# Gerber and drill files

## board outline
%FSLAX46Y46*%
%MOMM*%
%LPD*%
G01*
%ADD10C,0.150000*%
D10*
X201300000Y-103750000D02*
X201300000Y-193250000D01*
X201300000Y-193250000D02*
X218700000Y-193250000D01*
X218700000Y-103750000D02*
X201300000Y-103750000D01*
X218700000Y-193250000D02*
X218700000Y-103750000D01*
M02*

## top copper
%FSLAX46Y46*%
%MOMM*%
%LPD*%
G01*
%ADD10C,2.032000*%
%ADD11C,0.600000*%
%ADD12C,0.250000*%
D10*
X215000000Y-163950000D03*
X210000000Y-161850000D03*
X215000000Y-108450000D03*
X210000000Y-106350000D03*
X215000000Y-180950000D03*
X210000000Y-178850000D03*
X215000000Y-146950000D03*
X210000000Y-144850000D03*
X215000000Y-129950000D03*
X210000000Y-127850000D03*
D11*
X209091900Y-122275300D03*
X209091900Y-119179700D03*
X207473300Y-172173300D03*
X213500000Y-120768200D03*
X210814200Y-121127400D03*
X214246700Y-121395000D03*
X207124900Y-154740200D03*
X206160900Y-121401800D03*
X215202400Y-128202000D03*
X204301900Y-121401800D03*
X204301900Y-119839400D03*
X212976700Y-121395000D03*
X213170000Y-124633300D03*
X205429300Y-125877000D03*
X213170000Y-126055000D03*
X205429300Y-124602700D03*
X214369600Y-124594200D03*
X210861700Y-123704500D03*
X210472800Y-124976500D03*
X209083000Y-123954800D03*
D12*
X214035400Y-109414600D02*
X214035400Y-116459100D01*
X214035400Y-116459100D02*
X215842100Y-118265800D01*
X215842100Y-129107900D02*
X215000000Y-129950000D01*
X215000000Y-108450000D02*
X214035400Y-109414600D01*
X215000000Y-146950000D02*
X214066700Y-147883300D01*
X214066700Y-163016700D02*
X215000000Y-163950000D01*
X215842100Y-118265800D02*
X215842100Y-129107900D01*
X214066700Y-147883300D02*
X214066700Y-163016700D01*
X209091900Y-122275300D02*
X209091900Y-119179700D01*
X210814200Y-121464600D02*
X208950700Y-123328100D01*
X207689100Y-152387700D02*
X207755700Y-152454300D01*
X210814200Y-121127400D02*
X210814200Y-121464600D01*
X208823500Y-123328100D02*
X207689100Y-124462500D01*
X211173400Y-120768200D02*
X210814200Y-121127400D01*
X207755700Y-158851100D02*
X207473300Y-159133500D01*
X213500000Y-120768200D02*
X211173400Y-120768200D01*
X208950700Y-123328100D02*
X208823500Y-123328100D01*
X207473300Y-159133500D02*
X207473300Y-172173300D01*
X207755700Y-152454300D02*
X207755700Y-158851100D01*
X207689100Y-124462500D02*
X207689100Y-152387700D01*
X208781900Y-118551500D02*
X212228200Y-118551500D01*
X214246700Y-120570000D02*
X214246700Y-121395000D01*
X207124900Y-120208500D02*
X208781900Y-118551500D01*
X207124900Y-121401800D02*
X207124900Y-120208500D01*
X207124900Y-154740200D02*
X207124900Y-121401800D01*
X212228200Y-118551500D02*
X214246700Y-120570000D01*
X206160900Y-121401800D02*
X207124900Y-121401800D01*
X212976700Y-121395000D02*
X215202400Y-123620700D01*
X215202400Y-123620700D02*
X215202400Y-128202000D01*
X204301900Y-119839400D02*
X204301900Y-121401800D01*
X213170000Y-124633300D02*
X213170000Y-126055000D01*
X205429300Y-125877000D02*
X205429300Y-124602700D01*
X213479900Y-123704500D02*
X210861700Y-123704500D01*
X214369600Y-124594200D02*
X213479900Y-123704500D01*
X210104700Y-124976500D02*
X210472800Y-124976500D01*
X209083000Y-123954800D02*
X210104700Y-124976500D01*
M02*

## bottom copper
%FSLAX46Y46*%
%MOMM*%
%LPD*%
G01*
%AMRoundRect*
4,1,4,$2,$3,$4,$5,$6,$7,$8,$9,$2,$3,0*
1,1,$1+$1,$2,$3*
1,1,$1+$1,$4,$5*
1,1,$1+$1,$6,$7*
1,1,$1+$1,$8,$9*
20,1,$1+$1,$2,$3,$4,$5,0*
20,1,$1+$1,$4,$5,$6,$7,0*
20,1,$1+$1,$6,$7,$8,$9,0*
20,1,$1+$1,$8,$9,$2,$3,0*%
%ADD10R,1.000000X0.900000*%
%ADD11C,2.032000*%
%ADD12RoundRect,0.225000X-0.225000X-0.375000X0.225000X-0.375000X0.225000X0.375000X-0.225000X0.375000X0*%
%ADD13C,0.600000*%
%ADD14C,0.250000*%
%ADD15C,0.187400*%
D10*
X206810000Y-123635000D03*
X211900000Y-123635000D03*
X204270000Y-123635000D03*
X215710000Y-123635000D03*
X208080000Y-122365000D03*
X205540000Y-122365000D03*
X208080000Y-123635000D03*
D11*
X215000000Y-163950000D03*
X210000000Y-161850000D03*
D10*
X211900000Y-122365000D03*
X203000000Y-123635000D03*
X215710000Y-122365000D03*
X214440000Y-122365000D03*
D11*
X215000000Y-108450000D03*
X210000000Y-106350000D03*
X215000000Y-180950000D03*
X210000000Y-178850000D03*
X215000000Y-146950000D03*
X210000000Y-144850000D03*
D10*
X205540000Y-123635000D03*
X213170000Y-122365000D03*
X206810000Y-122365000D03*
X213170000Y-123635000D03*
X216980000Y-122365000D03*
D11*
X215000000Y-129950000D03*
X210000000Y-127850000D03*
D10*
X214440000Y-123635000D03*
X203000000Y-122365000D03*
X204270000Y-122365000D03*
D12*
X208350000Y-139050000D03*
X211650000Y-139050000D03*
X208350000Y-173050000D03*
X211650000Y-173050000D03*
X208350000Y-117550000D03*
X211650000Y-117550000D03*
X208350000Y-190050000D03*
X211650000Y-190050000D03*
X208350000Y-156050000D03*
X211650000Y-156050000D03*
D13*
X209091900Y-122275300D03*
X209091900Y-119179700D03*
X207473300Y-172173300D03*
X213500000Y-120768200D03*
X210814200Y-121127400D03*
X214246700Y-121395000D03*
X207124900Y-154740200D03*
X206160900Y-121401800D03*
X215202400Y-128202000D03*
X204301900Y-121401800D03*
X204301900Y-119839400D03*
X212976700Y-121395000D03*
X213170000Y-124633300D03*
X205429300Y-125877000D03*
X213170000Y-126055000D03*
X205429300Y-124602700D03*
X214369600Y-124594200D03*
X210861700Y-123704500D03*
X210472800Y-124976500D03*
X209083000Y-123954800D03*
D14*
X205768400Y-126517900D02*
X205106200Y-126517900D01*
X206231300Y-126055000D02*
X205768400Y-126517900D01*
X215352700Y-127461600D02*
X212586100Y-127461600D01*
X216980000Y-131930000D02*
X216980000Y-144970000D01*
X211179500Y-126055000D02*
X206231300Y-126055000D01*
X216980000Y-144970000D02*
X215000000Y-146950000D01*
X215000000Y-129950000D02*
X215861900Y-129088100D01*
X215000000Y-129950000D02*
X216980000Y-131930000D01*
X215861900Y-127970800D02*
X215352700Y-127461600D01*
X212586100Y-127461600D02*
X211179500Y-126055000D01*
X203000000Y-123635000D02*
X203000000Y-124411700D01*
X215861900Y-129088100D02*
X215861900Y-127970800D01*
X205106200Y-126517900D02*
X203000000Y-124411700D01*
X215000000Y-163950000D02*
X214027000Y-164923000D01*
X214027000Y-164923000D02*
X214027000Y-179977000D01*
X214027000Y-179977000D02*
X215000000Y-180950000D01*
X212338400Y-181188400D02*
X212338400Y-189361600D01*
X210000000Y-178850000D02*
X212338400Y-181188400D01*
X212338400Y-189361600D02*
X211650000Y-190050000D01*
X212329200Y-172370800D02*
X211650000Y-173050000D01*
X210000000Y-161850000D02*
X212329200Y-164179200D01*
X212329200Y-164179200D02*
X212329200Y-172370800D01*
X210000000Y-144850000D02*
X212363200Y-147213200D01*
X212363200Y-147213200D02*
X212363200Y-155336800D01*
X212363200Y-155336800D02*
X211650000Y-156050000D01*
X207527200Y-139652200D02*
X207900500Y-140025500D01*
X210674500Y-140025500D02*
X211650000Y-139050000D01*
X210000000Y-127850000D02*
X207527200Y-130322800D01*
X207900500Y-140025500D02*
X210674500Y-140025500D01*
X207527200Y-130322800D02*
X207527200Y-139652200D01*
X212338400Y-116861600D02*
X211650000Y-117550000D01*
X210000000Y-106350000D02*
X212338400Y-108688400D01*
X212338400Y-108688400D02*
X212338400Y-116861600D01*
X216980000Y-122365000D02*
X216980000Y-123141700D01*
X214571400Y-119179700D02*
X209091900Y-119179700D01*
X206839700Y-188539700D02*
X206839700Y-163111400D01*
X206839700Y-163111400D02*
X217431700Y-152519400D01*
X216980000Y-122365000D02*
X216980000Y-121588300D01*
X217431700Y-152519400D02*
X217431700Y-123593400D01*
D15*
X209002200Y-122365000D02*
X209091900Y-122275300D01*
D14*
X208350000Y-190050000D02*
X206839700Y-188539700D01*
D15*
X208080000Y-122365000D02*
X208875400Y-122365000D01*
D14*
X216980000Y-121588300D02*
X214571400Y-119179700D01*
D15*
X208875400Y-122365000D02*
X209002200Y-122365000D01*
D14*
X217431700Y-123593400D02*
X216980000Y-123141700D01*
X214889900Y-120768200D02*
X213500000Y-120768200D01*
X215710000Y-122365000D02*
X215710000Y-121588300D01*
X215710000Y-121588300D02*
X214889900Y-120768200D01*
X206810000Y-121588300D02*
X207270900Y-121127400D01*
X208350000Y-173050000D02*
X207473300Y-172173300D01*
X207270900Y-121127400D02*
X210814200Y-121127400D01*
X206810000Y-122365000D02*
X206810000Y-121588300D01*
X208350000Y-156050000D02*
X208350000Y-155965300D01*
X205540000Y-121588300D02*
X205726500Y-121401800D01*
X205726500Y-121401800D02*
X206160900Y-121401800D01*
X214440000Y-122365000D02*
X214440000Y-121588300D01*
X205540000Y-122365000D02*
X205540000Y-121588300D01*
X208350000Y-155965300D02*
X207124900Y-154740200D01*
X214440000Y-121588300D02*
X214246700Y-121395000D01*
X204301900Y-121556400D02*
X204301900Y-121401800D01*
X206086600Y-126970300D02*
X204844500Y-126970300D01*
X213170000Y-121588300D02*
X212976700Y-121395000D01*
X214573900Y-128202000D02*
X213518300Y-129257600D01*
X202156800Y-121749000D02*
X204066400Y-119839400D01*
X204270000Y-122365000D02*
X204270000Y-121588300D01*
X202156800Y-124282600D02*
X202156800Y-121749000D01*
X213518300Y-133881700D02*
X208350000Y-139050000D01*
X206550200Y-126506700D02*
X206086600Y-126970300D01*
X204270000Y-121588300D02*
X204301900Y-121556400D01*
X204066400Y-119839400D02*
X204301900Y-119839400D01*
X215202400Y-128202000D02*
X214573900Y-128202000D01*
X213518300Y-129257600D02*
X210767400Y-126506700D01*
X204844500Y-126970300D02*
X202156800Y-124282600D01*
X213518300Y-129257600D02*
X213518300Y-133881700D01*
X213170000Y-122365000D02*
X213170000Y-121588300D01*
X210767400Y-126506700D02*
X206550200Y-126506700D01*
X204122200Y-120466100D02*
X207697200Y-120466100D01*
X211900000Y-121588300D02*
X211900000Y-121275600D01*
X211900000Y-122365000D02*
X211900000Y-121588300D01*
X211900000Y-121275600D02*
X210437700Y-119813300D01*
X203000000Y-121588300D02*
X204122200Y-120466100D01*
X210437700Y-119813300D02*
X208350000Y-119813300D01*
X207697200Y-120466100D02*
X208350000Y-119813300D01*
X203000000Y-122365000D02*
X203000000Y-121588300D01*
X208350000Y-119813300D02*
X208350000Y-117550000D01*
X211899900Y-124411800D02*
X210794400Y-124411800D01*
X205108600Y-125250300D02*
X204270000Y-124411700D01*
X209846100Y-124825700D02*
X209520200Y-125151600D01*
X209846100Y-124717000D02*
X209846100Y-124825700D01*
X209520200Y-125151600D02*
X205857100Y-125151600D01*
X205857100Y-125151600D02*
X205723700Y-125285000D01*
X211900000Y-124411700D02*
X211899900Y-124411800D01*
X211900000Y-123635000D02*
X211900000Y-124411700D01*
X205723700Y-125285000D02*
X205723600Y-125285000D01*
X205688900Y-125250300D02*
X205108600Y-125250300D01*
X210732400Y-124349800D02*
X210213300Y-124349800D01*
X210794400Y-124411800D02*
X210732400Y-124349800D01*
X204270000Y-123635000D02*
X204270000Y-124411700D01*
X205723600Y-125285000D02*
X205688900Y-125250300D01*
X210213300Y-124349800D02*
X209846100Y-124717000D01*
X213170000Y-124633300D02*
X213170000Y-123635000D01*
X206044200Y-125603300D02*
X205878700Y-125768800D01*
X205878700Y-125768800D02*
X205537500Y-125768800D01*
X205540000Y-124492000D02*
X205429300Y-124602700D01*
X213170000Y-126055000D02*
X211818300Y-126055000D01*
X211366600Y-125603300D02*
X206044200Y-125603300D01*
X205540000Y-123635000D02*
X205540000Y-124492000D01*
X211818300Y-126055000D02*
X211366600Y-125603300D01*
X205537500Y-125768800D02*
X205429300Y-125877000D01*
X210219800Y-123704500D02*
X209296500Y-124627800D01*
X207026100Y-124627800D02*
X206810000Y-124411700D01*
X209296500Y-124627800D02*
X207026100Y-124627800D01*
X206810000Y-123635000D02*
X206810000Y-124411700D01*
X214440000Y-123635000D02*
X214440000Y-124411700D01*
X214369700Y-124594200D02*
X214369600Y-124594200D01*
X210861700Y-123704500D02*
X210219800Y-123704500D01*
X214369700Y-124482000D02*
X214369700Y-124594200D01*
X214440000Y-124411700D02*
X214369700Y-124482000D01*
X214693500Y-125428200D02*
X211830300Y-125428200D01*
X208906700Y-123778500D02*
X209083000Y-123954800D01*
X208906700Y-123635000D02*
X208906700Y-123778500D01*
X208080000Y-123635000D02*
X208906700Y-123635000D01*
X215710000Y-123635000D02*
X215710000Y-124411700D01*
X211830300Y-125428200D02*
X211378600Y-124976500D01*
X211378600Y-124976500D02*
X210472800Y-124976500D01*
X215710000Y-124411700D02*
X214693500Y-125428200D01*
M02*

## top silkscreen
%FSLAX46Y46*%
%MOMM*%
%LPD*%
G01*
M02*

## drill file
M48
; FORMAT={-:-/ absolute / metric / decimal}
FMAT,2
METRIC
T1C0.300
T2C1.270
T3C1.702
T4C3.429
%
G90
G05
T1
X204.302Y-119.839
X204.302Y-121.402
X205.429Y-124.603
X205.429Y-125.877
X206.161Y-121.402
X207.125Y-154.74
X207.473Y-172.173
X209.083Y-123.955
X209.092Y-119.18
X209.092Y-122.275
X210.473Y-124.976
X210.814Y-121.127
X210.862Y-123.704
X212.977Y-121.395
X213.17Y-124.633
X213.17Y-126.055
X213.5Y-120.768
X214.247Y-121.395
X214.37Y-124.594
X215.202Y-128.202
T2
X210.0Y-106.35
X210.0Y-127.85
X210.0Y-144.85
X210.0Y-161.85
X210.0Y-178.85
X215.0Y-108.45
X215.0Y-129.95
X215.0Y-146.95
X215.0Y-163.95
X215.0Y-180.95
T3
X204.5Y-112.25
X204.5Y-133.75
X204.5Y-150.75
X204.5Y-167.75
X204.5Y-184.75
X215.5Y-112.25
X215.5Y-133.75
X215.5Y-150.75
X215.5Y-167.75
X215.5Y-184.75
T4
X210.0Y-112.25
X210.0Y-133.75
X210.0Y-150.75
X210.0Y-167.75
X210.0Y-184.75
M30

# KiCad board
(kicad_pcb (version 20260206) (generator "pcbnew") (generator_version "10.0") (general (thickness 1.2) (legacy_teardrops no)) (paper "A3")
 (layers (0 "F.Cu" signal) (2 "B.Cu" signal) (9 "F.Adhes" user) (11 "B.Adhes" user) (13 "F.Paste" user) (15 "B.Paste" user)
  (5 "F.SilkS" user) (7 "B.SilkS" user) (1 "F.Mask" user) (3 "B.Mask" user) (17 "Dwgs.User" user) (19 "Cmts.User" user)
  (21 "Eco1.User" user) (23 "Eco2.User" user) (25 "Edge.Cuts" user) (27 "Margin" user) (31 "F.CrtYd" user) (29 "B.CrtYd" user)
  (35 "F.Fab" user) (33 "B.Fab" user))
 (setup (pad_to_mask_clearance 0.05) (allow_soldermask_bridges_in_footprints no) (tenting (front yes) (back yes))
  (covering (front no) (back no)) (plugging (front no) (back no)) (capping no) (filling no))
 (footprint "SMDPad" (layer "F.Cu") (at 206.81 123.635)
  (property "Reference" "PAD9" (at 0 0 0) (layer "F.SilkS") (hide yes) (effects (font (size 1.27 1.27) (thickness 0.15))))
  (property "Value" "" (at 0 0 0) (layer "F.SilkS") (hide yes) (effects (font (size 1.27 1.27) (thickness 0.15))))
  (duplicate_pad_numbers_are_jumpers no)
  (pad "1" smd rect (at 0 0) (size 1 0.9) (layers "B.Cu" "B.Mask" "B.Paste") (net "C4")))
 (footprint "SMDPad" (layer "F.Cu") (at 211.9 123.635)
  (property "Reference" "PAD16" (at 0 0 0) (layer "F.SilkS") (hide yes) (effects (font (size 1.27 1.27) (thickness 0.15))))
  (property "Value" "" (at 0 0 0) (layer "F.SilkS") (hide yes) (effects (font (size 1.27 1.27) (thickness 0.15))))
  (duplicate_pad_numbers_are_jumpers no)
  (pad "1" smd rect (at 0 0) (size 1 0.9) (layers "B.Cu" "B.Mask" "B.Paste") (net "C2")))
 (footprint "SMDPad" (layer "F.Cu") (at 204.27 123.635)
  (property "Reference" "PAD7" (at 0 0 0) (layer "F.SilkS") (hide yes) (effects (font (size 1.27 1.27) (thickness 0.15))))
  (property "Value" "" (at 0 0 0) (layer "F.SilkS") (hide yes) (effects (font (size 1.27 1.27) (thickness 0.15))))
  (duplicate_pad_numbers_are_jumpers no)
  (pad "1" smd rect (at 0 0) (size 1 0.9) (layers "B.Cu" "B.Mask" "B.Paste") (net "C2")))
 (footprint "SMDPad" (layer "F.Cu") (at 215.71 123.635)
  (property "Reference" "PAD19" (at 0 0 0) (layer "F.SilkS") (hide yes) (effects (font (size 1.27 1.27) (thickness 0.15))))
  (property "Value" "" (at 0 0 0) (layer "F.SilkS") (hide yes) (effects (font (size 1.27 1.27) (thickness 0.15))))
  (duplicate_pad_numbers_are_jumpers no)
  (pad "1" smd rect (at 0 0) (size 1 0.9) (layers "B.Cu" "B.Mask" "B.Paste") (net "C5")))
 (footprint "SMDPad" (layer "F.Cu") (at 208.08 122.365)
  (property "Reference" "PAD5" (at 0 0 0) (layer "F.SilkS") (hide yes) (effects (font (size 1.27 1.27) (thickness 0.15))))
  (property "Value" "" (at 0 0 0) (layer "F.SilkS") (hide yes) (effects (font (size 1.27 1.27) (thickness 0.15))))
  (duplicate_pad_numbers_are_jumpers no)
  (pad "1" smd rect (at 0 0) (size 1 0.9) (layers "B.Cu" "B.Mask" "B.Paste") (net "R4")))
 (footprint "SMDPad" (layer "F.Cu") (at 205.54 122.365)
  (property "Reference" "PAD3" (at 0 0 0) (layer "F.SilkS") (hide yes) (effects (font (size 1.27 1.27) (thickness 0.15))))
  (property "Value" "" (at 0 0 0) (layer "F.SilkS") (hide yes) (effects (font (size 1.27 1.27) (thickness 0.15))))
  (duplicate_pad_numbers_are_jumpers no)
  (pad "1" smd rect (at 0 0) (size 1 0.9) (layers "B.Cu" "B.Mask" "B.Paste") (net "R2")))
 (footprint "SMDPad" (layer "F.Cu") (at 208.08 123.635)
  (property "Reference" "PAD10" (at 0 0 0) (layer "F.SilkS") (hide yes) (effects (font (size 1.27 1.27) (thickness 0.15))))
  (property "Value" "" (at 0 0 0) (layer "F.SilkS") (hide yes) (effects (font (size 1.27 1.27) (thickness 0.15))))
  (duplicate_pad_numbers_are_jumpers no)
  (pad "1" smd rect (at 0 0) (size 1 0.9) (layers "B.Cu" "B.Mask" "B.Paste") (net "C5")))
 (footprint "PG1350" (layer "F.Cu") (at 210 167.75)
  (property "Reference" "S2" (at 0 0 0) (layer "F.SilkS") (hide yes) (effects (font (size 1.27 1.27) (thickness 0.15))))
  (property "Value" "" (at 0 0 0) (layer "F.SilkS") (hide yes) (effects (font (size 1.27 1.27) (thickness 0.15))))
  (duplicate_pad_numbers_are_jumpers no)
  (pad "" np_thru_hole circle (at -5.5 0) (size 1.7018 1.7018) (drill 1.7018) (layers "*.Cu" "*.Mask"))
  (pad "" np_thru_hole circle (at 0 0) (size 3.429 3.429) (drill 3.429) (layers "*.Cu" "*.Mask"))
  (pad "" np_thru_hole circle (at 5.5 0) (size 1.7018 1.7018) (drill 1.7018) (layers "*.Cu" "*.Mask"))
  (pad "1" thru_hole circle (at 5 -3.8) (size 2.032 2.032) (drill 1.27) (layers "*.Cu" "*.Mask") (remove_unused_layers no) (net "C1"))
  (pad "2" thru_hole circle (at 0 -5.9) (size 2.032 2.032) (drill 1.27) (layers "*.Cu" "*.Mask") (remove_unused_layers no) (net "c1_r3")))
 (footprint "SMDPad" (layer "F.Cu") (at 211.9 122.365)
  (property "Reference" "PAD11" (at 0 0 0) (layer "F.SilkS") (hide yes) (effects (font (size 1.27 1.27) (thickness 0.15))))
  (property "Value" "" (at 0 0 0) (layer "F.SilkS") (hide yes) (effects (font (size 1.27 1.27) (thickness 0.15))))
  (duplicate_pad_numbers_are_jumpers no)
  (pad "1" smd rect (at 0 0) (size 1 0.9) (layers "B.Cu" "B.Mask" "B.Paste") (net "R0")))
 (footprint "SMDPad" (layer "F.Cu") (at 203 123.635)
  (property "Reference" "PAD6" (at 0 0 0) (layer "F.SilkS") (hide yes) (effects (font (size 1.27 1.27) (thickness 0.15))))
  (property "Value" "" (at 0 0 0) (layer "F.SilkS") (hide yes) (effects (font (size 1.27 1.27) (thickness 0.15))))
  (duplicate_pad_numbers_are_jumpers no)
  (pad "1" smd rect (at 0 0) (size 1 0.9) (layers "B.Cu" "B.Mask" "B.Paste") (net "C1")))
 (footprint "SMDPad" (layer "F.Cu") (at 215.71 122.365)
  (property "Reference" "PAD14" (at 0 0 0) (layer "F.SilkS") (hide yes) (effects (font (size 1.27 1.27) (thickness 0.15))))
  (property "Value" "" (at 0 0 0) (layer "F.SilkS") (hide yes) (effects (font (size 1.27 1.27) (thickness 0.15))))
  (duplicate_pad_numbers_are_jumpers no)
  (pad "1" smd rect (at 0 0) (size 1 0.9) (layers "B.Cu" "B.Mask" "B.Paste") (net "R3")))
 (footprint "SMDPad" (layer "F.Cu") (at 214.44 122.365)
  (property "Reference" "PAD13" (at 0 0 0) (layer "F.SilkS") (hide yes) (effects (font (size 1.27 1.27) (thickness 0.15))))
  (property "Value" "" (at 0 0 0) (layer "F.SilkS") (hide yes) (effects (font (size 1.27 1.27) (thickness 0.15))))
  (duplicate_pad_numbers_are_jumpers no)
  (pad "1" smd rect (at 0 0) (size 1 0.9) (layers "B.Cu" "B.Mask" "B.Paste") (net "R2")))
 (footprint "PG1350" (layer "F.Cu") (at 210 112.25)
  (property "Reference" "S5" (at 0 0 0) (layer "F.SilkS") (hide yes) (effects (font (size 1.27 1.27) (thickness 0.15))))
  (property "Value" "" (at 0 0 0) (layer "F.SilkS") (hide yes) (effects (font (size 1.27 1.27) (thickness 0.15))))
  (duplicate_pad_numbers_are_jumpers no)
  (pad "" np_thru_hole circle (at -5.5 0) (size 1.7018 1.7018) (drill 1.7018) (layers "*.Cu" "*.Mask"))
  (pad "" np_thru_hole circle (at 0 0) (size 3.429 3.429) (drill 3.429) (layers "*.Cu" "*.Mask"))
  (pad "" np_thru_hole circle (at 5.5 0) (size 1.7018 1.7018) (drill 1.7018) (layers "*.Cu" "*.Mask"))
  (pad "1" thru_hole circle (at 5 -3.8) (size 2.032 2.032) (drill 1.27) (layers "*.Cu" "*.Mask") (remove_unused_layers no) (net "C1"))
  (pad "2" thru_hole circle (at 0 -5.9) (size 2.032 2.032) (drill 1.27) (layers "*.Cu" "*.Mask") (remove_unused_layers no) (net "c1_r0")))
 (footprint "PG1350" (layer "F.Cu") (at 210 184.75)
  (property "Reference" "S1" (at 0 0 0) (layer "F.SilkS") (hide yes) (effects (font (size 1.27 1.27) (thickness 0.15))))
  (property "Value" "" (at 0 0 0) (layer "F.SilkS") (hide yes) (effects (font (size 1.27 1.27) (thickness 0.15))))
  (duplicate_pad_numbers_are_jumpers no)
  (pad "" np_thru_hole circle (at -5.5 0) (size 1.7018 1.7018) (drill 1.7018) (layers "*.Cu" "*.Mask"))
  (pad "" np_thru_hole circle (at 0 0) (size 3.429 3.429) (drill 3.429) (layers "*.Cu" "*.Mask"))
  (pad "" np_thru_hole circle (at 5.5 0) (size 1.7018 1.7018) (drill 1.7018) (layers "*.Cu" "*.Mask"))
  (pad "1" thru_hole circle (at 5 -3.8) (size 2.032 2.032) (drill 1.27) (layers "*.Cu" "*.Mask") (remove_unused_layers no) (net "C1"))
  (pad "2" thru_hole circle (at 0 -5.9) (size 2.032 2.032) (drill 1.27) (layers "*.Cu" "*.Mask") (remove_unused_layers no) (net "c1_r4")))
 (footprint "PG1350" (layer "F.Cu") (at 210 150.75)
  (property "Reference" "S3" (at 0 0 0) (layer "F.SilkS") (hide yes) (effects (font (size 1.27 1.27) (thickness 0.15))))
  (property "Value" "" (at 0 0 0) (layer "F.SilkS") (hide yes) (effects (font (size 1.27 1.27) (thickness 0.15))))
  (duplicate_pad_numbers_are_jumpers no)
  (pad "" np_thru_hole circle (at -5.5 0) (size 1.7018 1.7018) (drill 1.7018) (layers "*.Cu" "*.Mask"))
  (pad "" np_thru_hole circle (at 0 0) (size 3.429 3.429) (drill 3.429) (layers "*.Cu" "*.Mask"))
  (pad "" np_thru_hole circle (at 5.5 0) (size 1.7018 1.7018) (drill 1.7018) (layers "*.Cu" "*.Mask"))
  (pad "1" thru_hole circle (at 5 -3.8) (size 2.032 2.032) (drill 1.27) (layers "*.Cu" "*.Mask") (remove_unused_layers no) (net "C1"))
  (pad "2" thru_hole circle (at 0 -5.9) (size 2.032 2.032) (drill 1.27) (layers "*.Cu" "*.Mask") (remove_unused_layers no) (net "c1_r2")))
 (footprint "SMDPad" (layer "F.Cu") (at 205.54 123.635)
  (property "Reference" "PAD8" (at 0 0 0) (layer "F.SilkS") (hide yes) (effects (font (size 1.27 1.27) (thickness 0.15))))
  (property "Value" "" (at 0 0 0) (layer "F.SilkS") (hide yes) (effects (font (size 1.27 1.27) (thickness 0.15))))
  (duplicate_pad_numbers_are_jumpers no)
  (pad "1" smd rect (at 0 0) (size 1 0.9) (layers "B.Cu" "B.Mask" "B.Paste") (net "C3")))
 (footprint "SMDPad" (layer "F.Cu") (at 213.17 122.365)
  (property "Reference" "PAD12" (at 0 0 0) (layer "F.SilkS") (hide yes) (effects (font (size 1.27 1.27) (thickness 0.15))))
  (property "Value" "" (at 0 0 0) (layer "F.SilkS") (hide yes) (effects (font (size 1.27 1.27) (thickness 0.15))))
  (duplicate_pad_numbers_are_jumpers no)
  (pad "1" smd rect (at 0 0) (size 1 0.9) (layers "B.Cu" "B.Mask" "B.Paste") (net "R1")))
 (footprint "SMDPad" (layer "F.Cu") (at 206.81 122.365)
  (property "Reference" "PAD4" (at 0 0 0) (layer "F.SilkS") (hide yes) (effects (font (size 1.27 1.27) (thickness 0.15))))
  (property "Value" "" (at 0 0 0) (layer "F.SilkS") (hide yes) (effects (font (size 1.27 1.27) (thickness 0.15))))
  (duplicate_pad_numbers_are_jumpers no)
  (pad "1" smd rect (at 0 0) (size 1 0.9) (layers "B.Cu" "B.Mask" "B.Paste") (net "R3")))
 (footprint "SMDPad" (layer "F.Cu") (at 213.17 123.635)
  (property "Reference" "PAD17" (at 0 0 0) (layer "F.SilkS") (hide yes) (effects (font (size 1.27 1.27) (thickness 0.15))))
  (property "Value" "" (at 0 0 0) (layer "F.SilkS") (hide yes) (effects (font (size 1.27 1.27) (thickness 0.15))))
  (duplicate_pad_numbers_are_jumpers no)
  (pad "1" smd rect (at 0 0) (size 1 0.9) (layers "B.Cu" "B.Mask" "B.Paste") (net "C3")))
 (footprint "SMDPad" (layer "F.Cu") (at 216.98 122.365)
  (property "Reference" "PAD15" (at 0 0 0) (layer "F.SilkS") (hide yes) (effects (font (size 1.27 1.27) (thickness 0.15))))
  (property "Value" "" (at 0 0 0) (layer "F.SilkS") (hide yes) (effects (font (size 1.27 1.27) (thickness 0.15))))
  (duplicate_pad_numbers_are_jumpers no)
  (pad "1" smd rect (at 0 0) (size 1 0.9) (layers "B.Cu" "B.Mask" "B.Paste") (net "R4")))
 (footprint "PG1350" (layer "F.Cu") (at 210 133.75)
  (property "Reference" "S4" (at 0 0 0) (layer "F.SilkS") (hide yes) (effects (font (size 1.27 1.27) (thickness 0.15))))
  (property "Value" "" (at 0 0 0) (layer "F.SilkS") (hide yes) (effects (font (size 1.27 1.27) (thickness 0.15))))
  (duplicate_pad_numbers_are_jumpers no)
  (pad "" np_thru_hole circle (at -5.5 0) (size 1.7018 1.7018) (drill 1.7018) (layers "*.Cu" "*.Mask"))
  (pad "" np_thru_hole circle (at 0 0) (size 3.429 3.429) (drill 3.429) (layers "*.Cu" "*.Mask"))
  (pad "" np_thru_hole circle (at 5.5 0) (size 1.7018 1.7018) (drill 1.7018) (layers "*.Cu" "*.Mask"))
  (pad "1" thru_hole circle (at 5 -3.8) (size 2.032 2.032) (drill 1.27) (layers "*.Cu" "*.Mask") (remove_unused_layers no) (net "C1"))
  (pad "2" thru_hole circle (at 0 -5.9) (size 2.032 2.032) (drill 1.27) (layers "*.Cu" "*.Mask") (remove_unused_layers no) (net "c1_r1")))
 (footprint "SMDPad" (layer "F.Cu") (at 214.44 123.635)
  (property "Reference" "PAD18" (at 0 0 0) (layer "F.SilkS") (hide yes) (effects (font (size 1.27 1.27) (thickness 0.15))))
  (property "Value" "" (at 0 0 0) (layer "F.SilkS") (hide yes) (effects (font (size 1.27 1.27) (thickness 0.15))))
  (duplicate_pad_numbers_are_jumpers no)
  (pad "1" smd rect (at 0 0) (size 1 0.9) (layers "B.Cu" "B.Mask" "B.Paste") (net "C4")))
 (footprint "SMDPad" (layer "F.Cu") (at 203 122.365)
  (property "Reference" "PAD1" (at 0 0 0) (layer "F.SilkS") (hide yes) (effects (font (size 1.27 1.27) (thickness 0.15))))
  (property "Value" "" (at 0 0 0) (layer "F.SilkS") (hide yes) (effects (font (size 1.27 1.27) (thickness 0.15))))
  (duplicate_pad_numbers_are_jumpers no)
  (pad "1" smd rect (at 0 0) (size 1 0.9) (layers "B.Cu" "B.Mask" "B.Paste") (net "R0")))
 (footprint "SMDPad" (layer "F.Cu") (at 204.27 122.365)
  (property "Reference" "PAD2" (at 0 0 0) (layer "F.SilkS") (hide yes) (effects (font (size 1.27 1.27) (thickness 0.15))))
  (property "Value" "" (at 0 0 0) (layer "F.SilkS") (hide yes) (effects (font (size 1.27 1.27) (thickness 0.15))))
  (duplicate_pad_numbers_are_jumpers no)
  (pad "1" smd rect (at 0 0) (size 1 0.9) (layers "B.Cu" "B.Mask" "B.Paste") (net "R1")))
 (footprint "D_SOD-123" (layer "B.Cu") (at 210 139.05)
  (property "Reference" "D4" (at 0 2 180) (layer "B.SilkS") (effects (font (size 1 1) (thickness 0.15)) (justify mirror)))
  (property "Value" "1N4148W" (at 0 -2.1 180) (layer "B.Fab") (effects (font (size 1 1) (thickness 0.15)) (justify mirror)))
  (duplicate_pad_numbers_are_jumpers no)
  (pad "1" smd roundrect (at -1.65 0) (size 0.9 1.2) (layers "B.Cu" "B.Mask" "B.Paste") (roundrect_rratio 0.25) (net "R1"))
  (pad "2" smd roundrect (at 1.65 0) (size 0.9 1.2) (layers "B.Cu" "B.Mask" "B.Paste") (roundrect_rratio 0.25) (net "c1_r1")))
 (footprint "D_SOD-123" (layer "B.Cu") (at 210 173.05)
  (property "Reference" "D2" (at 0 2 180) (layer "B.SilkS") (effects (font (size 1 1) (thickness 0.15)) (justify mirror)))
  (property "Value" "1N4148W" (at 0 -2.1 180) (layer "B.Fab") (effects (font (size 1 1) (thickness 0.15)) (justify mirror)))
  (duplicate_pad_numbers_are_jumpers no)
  (pad "1" smd roundrect (at -1.65 0) (size 0.9 1.2) (layers "B.Cu" "B.Mask" "B.Paste") (roundrect_rratio 0.25) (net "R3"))
  (pad "2" smd roundrect (at 1.65 0) (size 0.9 1.2) (layers "B.Cu" "B.Mask" "B.Paste") (roundrect_rratio 0.25) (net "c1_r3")))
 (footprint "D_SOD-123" (layer "B.Cu") (at 210 117.55)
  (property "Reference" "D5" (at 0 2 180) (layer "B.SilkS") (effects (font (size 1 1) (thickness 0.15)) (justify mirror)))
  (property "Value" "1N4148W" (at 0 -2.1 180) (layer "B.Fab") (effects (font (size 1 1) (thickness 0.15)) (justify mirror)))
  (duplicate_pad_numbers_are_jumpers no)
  (pad "1" smd roundrect (at -1.65 0) (size 0.9 1.2) (layers "B.Cu" "B.Mask" "B.Paste") (roundrect_rratio 0.25) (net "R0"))
  (pad "2" smd roundrect (at 1.65 0) (size 0.9 1.2) (layers "B.Cu" "B.Mask" "B.Paste") (roundrect_rratio 0.25) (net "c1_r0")))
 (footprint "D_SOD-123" (layer "B.Cu") (at 210 190.05)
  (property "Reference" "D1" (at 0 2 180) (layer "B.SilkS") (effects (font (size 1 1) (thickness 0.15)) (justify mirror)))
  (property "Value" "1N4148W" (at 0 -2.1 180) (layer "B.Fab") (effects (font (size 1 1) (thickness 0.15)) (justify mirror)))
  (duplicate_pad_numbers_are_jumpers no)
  (pad "1" smd roundrect (at -1.65 0) (size 0.9 1.2) (layers "B.Cu" "B.Mask" "B.Paste") (roundrect_rratio 0.25) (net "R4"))
  (pad "2" smd roundrect (at 1.65 0) (size 0.9 1.2) (layers "B.Cu" "B.Mask" "B.Paste") (roundrect_rratio 0.25) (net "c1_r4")))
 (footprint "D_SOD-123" (layer "B.Cu") (at 210 156.05)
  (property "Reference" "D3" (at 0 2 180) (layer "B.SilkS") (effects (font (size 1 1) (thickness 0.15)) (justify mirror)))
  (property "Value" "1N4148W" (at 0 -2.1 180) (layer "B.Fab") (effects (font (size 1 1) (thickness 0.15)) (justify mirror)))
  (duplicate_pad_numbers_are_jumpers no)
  (pad "1" smd roundrect (at -1.65 0) (size 0.9 1.2) (layers "B.Cu" "B.Mask" "B.Paste") (roundrect_rratio 0.25) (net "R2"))
  (pad "2" smd roundrect (at 1.65 0) (size 0.9 1.2) (layers "B.Cu" "B.Mask" "B.Paste") (roundrect_rratio 0.25) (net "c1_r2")))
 (gr_line (start 201.3 103.75) (end 201.3 193.25) (stroke (width 0.15) (type solid)) (layer "Edge.Cuts"))
 (gr_line (start 201.3 193.25) (end 218.7 193.25) (stroke (width 0.15) (type solid)) (layer "Edge.Cuts"))
 (gr_line (start 218.7 103.75) (end 201.3 103.75) (stroke (width 0.15) (type solid)) (layer "Edge.Cuts"))
 (gr_line (start 218.7 193.25) (end 218.7 103.75) (stroke (width 0.15) (type solid)) (layer "Edge.Cuts"))
 (segment (start 214.0354 109.4146) (end 214.0354 116.4591) (width 0.25) (layer "F.Cu") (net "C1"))
 (segment (start 214.0354 116.4591) (end 215.8421 118.2658) (width 0.25) (layer "F.Cu") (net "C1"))
 (segment (start 215.8421 129.1079) (end 215 129.95) (width 0.25) (layer "F.Cu") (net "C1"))
 (segment (start 215 108.45) (end 214.0354 109.4146) (width 0.25) (layer "F.Cu") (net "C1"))
 (segment (start 215 146.95) (end 214.0667 147.8833) (width 0.25) (layer "F.Cu") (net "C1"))
 (segment (start 214.0667 163.0167) (end 215 163.95) (width 0.25) (layer "F.Cu") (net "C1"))
 (segment (start 215.8421 118.2658) (end 215.8421 129.1079) (width 0.25) (layer "F.Cu") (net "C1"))
 (segment (start 214.0667 147.8833) (end 214.0667 163.0167) (width 0.25) (layer "F.Cu") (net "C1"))
 (segment (start 205.7684 126.5179) (end 205.1062 126.5179) (width 0.25) (layer "B.Cu") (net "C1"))
 (segment (start 206.2313 126.055) (end 205.7684 126.5179) (width 0.25) (layer "B.Cu") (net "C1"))
 (segment (start 215.3527 127.4616) (end 212.5861 127.4616) (width 0.25) (layer "B.Cu") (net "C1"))
 (segment (start 216.98 131.93) (end 216.98 144.97) (width 0.25) (layer "B.Cu") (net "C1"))
 (segment (start 211.1795 126.055) (end 206.2313 126.055) (width 0.25) (layer "B.Cu") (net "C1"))
 (segment (start 216.98 144.97) (end 215 146.95) (width 0.25) (layer "B.Cu") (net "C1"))
 (segment (start 215 129.95) (end 215.8619 129.0881) (width 0.25) (layer "B.Cu") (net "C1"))
 (segment (start 215 129.95) (end 216.98 131.93) (width 0.25) (layer "B.Cu") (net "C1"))
 (segment (start 215.8619 127.9708) (end 215.3527 127.4616) (width 0.25) (layer "B.Cu") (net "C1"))
 (segment (start 212.5861 127.4616) (end 211.1795 126.055) (width 0.25) (layer "B.Cu") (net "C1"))
 (segment (start 203 123.635) (end 203 124.4117) (width 0.25) (layer "B.Cu") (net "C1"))
 (segment (start 215.8619 129.0881) (end 215.8619 127.9708) (width 0.25) (layer "B.Cu") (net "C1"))
 (segment (start 205.1062 126.5179) (end 203 124.4117) (width 0.25) (layer "B.Cu") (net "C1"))
 (segment (start 215 163.95) (end 214.027 164.923) (width 0.25) (layer "B.Cu") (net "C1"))
 (segment (start 214.027 164.923) (end 214.027 179.977) (width 0.25) (layer "B.Cu") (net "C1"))
 (segment (start 214.027 179.977) (end 215 180.95) (width 0.25) (layer "B.Cu") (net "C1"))
 (segment (start 212.3384 181.1884) (end 212.3384 189.3616) (width 0.25) (layer "B.Cu") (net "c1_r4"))
 (segment (start 210 178.85) (end 212.3384 181.1884) (width 0.25) (layer "B.Cu") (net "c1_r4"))
 (segment (start 212.3384 189.3616) (end 211.65 190.05) (width 0.25) (layer "B.Cu") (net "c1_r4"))
 (segment (start 212.3292 172.3708) (end 211.65 173.05) (width 0.25) (layer "B.Cu") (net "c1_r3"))
 (segment (start 210 161.85) (end 212.3292 164.1792) (width 0.25) (layer "B.Cu") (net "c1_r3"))
 (segment (start 212.3292 164.1792) (end 212.3292 172.3708) (width 0.25) (layer "B.Cu") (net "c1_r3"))
 (segment (start 210 144.85) (end 212.3632 147.2132) (width 0.25) (layer "B.Cu") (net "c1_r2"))
 (segment (start 212.3632 147.2132) (end 212.3632 155.3368) (width 0.25) (layer "B.Cu") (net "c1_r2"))
 (segment (start 212.3632 155.3368) (end 211.65 156.05) (width 0.25) (layer "B.Cu") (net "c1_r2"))
 (segment (start 207.5272 139.6522) (end 207.9005 140.0255) (width 0.25) (layer "B.Cu") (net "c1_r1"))
 (segment (start 210.6745 140.0255) (end 211.65 139.05) (width 0.25) (layer "B.Cu") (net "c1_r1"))
 (segment (start 210 127.85) (end 207.5272 130.3228) (width 0.25) (layer "B.Cu") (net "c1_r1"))
 (segment (start 207.9005 140.0255) (end 210.6745 140.0255) (width 0.25) (layer "B.Cu") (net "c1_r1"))
 (segment (start 207.5272 130.3228) (end 207.5272 139.6522) (width 0.25) (layer "B.Cu") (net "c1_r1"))
 (segment (start 212.3384 116.8616) (end 211.65 117.55) (width 0.25) (layer "B.Cu") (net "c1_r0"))
 (segment (start 210 106.35) (end 212.3384 108.6884) (width 0.25) (layer "B.Cu") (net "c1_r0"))
 (segment (start 212.3384 108.6884) (end 212.3384 116.8616) (width 0.25) (layer "B.Cu") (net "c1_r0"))
 (segment (start 209.0919 122.2753) (end 209.0919 119.1797) (width 0.25) (layer "F.Cu") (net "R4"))
 (via (at 209.0919 122.2753) (size 0.6) (drill 0.3) (layers "F.Cu" "B.Cu") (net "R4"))
 (via (at 209.0919 119.1797) (size 0.6) (drill 0.3) (layers "F.Cu" "B.Cu") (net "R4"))
 (segment (start 216.98 122.365) (end 216.98 123.1417) (width 0.25) (layer "B.Cu") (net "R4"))
 (segment (start 214.5714 119.1797) (end 209.0919 119.1797) (width 0.25) (layer "B.Cu") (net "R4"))
 (segment (start 206.8397 188.5397) (end 206.8397 163.1114) (width 0.25) (layer "B.Cu") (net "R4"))
 (segment (start 206.8397 163.1114) (end 217.4317 152.5194) (width 0.25) (layer "B.Cu") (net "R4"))
 (segment (start 216.98 122.365) (end 216.98 121.5883) (width 0.25) (layer "B.Cu") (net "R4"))
 (segment (start 217.4317 152.5194) (end 217.4317 123.5934) (width 0.25) (layer "B.Cu") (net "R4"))
 (segment (start 209.0022 122.365) (end 209.0919 122.2753) (width 0.1874) (layer "B.Cu") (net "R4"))
 (segment (start 208.35 190.05) (end 206.8397 188.5397) (width 0.25) (layer "B.Cu") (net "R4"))
 (segment (start 208.08 122.365) (end 208.8754 122.365) (width 0.1874) (layer "B.Cu") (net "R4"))
 (segment (start 216.98 121.5883) (end 214.5714 119.1797) (width 0.25) (layer "B.Cu") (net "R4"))
 (segment (start 208.8754 122.365) (end 209.0022 122.365) (width 0.1874) (layer "B.Cu") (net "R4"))
 (segment (start 217.4317 123.5934) (end 216.98 123.1417) (width 0.25) (layer "B.Cu") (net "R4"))
 (segment (start 210.8142 121.4646) (end 208.9507 123.3281) (width 0.25) (layer "F.Cu") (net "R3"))
 (segment (start 207.6891 152.3877) (end 207.7557 152.4543) (width 0.25) (layer "F.Cu") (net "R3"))
 (segment (start 210.8142 121.1274) (end 210.8142 121.4646) (width 0.25) (layer "F.Cu") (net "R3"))
 (segment (start 208.8235 123.3281) (end 207.6891 124.4625) (width 0.25) (layer "F.Cu") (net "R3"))
 (segment (start 211.1734 120.7682) (end 210.8142 121.1274) (width 0.25) (layer "F.Cu") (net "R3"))
 (segment (start 207.7557 158.8511) (end 207.4733 159.1335) (width 0.25) (layer "F.Cu") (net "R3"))
 (segment (start 213.5 120.7682) (end 211.1734 120.7682) (width 0.25) (layer "F.Cu") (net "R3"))
 (segment (start 208.9507 123.3281) (end 208.8235 123.3281) (width 0.25) (layer "F.Cu") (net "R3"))
 (segment (start 207.4733 159.1335) (end 207.4733 172.1733) (width 0.25) (layer "F.Cu") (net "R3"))
 (segment (start 207.7557 152.4543) (end 207.7557 158.8511) (width 0.25) (layer "F.Cu") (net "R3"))
 (segment (start 207.6891 124.4625) (end 207.6891 152.3877) (width 0.25) (layer "F.Cu") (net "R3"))
 (via (at 207.4733 172.1733) (size 0.6) (drill 0.3) (layers "F.Cu" "B.Cu") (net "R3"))
 (via (at 213.5 120.7682) (size 0.6) (drill 0.3) (layers "F.Cu" "B.Cu") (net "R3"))
 (via (at 210.8142 121.1274) (size 0.6) (drill 0.3) (layers "F.Cu" "B.Cu") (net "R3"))
 (segment (start 214.8899 120.7682) (end 213.5 120.7682) (width 0.25) (layer "B.Cu") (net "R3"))
 (segment (start 215.71 122.365) (end 215.71 121.5883) (width 0.25) (layer "B.Cu") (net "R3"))
 (segment (start 215.71 121.5883) (end 214.8899 120.7682) (width 0.25) (layer "B.Cu") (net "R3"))
 (segment (start 206.81 121.5883) (end 207.2709 121.1274) (width 0.25) (layer "B.Cu") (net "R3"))
 (segment (start 208.35 173.05) (end 207.4733 172.1733) (width 0.25) (layer "B.Cu") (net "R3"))
 (segment (start 207.2709 121.1274) (end 210.8142 121.1274) (width 0.25) (layer "B.Cu") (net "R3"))
 (segment (start 206.81 122.365) (end 206.81 121.5883) (width 0.25) (layer "B.Cu") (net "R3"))
 (segment (start 208.7819 118.5515) (end 212.2282 118.5515) (width 0.25) (layer "F.Cu") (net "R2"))
 (segment (start 214.2467 120.57) (end 214.2467 121.395) (width 0.25) (layer "F.Cu") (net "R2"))
 (segment (start 207.1249 120.2085) (end 208.7819 118.5515) (width 0.25) (layer "F.Cu") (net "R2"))
 (segment (start 207.1249 121.4018) (end 207.1249 120.2085) (width 0.25) (layer "F.Cu") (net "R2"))
 (segment (start 207.1249 154.7402) (end 207.1249 121.4018) (width 0.25) (layer "F.Cu") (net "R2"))
 (segment (start 212.2282 118.5515) (end 214.2467 120.57) (width 0.25) (layer "F.Cu") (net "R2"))
 (segment (start 206.1609 121.4018) (end 207.1249 121.4018) (width 0.25) (layer "F.Cu") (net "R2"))
 (via (at 214.2467 121.395) (size 0.6) (drill 0.3) (layers "F.Cu" "B.Cu") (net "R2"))
 (via (at 207.1249 154.7402) (size 0.6) (drill 0.3) (layers "F.Cu" "B.Cu") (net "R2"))
 (via (at 206.1609 121.4018) (size 0.6) (drill 0.3) (layers "F.Cu" "B.Cu") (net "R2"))
 (segment (start 208.35 156.05) (end 208.35 155.9653) (width 0.25) (layer "B.Cu") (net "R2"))
 (segment (start 205.54 121.5883) (end 205.7265 121.4018) (width 0.25) (layer "B.Cu") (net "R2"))
 (segment (start 205.7265 121.4018) (end 206.1609 121.4018) (width 0.25) (layer "B.Cu") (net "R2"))
 (segment (start 214.44 122.365) (end 214.44 121.5883) (width 0.25) (layer "B.Cu") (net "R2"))
 (segment (start 205.54 122.365) (end 205.54 121.5883) (width 0.25) (layer "B.Cu") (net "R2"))
 (segment (start 208.35 155.9653) (end 207.1249 154.7402) (width 0.25) (layer "B.Cu") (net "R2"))
 (segment (start 214.44 121.5883) (end 214.2467 121.395) (width 0.25) (layer "B.Cu") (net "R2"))
 (segment (start 212.9767 121.395) (end 215.2024 123.6207) (width 0.25) (layer "F.Cu") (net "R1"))
 (segment (start 215.2024 123.6207) (end 215.2024 128.202) (width 0.25) (layer "F.Cu") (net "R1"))
 (segment (start 204.3019 119.8394) (end 204.3019 121.4018) (width 0.25) (layer "F.Cu") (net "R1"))
 (via (at 215.2024 128.202) (size 0.6) (drill 0.3) (layers "F.Cu" "B.Cu") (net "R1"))
 (via (at 204.3019 121.4018) (size 0.6) (drill 0.3) (layers "F.Cu" "B.Cu") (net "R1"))
 (via (at 204.3019 119.8394) (size 0.6) (drill 0.3) (layers "F.Cu" "B.Cu") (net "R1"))
 (via (at 212.9767 121.395) (size 0.6) (drill 0.3) (layers "F.Cu" "B.Cu") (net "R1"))
 (segment (start 204.3019 121.5564) (end 204.3019 121.4018) (width 0.25) (layer "B.Cu") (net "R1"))
 (segment (start 206.0866 126.9703) (end 204.8445 126.9703) (width 0.25) (layer "B.Cu") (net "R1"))
 (segment (start 213.17 121.5883) (end 212.9767 121.395) (width 0.25) (layer "B.Cu") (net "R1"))
 (segment (start 214.5739 128.202) (end 213.5183 129.2576) (width 0.25) (layer "B.Cu") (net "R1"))
 (segment (start 202.1568 121.749) (end 204.0664 119.8394) (width 0.25) (layer "B.Cu") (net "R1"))
 (segment (start 204.27 122.365) (end 204.27 121.5883) (width 0.25) (layer "B.Cu") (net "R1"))
 (segment (start 202.1568 124.2826) (end 202.1568 121.749) (width 0.25) (layer "B.Cu") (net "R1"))
 (segment (start 213.5183 133.8817) (end 208.35 139.05) (width 0.25) (layer "B.Cu") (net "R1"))
 (segment (start 206.5502 126.5067) (end 206.0866 126.9703) (width 0.25) (layer "B.Cu") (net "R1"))
 (segment (start 204.27 121.5883) (end 204.3019 121.5564) (width 0.25) (layer "B.Cu") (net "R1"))
 (segment (start 204.0664 119.8394) (end 204.3019 119.8394) (width 0.25) (layer "B.Cu") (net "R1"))
 (segment (start 215.2024 128.202) (end 214.5739 128.202) (width 0.25) (layer "B.Cu") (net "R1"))
 (segment (start 213.5183 129.2576) (end 210.7674 126.5067) (width 0.25) (layer "B.Cu") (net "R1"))
 (segment (start 204.8445 126.9703) (end 202.1568 124.2826) (width 0.25) (layer "B.Cu") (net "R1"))
 (segment (start 213.5183 129.2576) (end 213.5183 133.8817) (width 0.25) (layer "B.Cu") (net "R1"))
 (segment (start 213.17 122.365) (end 213.17 121.5883) (width 0.25) (layer "B.Cu") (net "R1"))
 (segment (start 210.7674 126.5067) (end 206.5502 126.5067) (width 0.25) (layer "B.Cu") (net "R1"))
 (segment (start 204.1222 120.4661) (end 207.6972 120.4661) (width 0.25) (layer "B.Cu") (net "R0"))
 (segment (start 211.9 121.5883) (end 211.9 121.2756) (width 0.25) (layer "B.Cu") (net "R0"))
 (segment (start 211.9 122.365) (end 211.9 121.5883) (width 0.25) (layer "B.Cu") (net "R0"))
 (segment (start 211.9 121.2756) (end 210.4377 119.8133) (width 0.25) (layer "B.Cu") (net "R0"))
 (segment (start 203 121.5883) (end 204.1222 120.4661) (width 0.25) (layer "B.Cu") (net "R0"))
 (segment (start 210.4377 119.8133) (end 208.35 119.8133) (width 0.25) (layer "B.Cu") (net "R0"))
 (segment (start 207.6972 120.4661) (end 208.35 119.8133) (width 0.25) (layer "B.Cu") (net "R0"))
 (segment (start 203 122.365) (end 203 121.5883) (width 0.25) (layer "B.Cu") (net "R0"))
 (segment (start 208.35 119.8133) (end 208.35 117.55) (width 0.25) (layer "B.Cu") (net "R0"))
 (segment (start 211.8999 124.4118) (end 210.7944 124.4118) (width 0.25) (layer "B.Cu") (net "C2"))
 (segment (start 205.1086 125.2503) (end 204.27 124.4117) (width 0.25) (layer "B.Cu") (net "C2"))
 (segment (start 209.8461 124.8257) (end 209.5202 125.1516) (width 0.25) (layer "B.Cu") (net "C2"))
 (segment (start 209.8461 124.717) (end 209.8461 124.8257) (width 0.25) (layer "B.Cu") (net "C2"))
 (segment (start 209.5202 125.1516) (end 205.8571 125.1516) (width 0.25) (layer "B.Cu") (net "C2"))
 (segment (start 205.8571 125.1516) (end 205.7237 125.285) (width 0.25) (layer "B.Cu") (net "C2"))
 (segment (start 211.9 124.4117) (end 211.8999 124.4118) (width 0.25) (layer "B.Cu") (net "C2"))
 (segment (start 211.9 123.635) (end 211.9 124.4117) (width 0.25) (layer "B.Cu") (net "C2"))
 (segment (start 205.7237 125.285) (end 205.7236 125.285) (width 0.25) (layer "B.Cu") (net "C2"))
 (segment (start 205.6889 125.2503) (end 205.1086 125.2503) (width 0.25) (layer "B.Cu") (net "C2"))
 (segment (start 210.7324 124.3498) (end 210.2133 124.3498) (width 0.25) (layer "B.Cu") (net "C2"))
 (segment (start 210.7944 124.4118) (end 210.7324 124.3498) (width 0.25) (layer "B.Cu") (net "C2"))
 (segment (start 204.27 123.635) (end 204.27 124.4117) (width 0.25) (layer "B.Cu") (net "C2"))
 (segment (start 205.7236 125.285) (end 205.6889 125.2503) (width 0.25) (layer "B.Cu") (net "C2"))
 (segment (start 210.2133 124.3498) (end 209.8461 124.717) (width 0.25) (layer "B.Cu") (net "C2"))
 (segment (start 213.17 124.6333) (end 213.17 126.055) (width 0.25) (layer "F.Cu") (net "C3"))
 (segment (start 205.4293 125.877) (end 205.4293 124.6027) (width 0.25) (layer "F.Cu") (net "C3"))
 (via (at 213.17 124.6333) (size 0.6) (drill 0.3) (layers "F.Cu" "B.Cu") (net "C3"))
 (via (at 205.4293 125.877) (size 0.6) (drill 0.3) (layers "F.Cu" "B.Cu") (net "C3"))
 (via (at 213.17 126.055) (size 0.6) (drill 0.3) (layers "F.Cu" "B.Cu") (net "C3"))
 (via (at 205.4293 124.6027) (size 0.6) (drill 0.3) (layers "F.Cu" "B.Cu") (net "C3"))
 (segment (start 213.17 124.6333) (end 213.17 123.635) (width 0.25) (layer "B.Cu") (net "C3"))
 (segment (start 206.0442 125.6033) (end 205.8787 125.7688) (width 0.25) (layer "B.Cu") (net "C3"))
 (segment (start 205.8787 125.7688) (end 205.5375 125.7688) (width 0.25) (layer "B.Cu") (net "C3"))
 (segment (start 205.54 124.492) (end 205.4293 124.6027) (width 0.25) (layer "B.Cu") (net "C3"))
 (segment (start 213.17 126.055) (end 211.8183 126.055) (width 0.25) (layer "B.Cu") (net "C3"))
 (segment (start 211.3666 125.6033) (end 206.0442 125.6033) (width 0.25) (layer "B.Cu") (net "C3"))
 (segment (start 205.54 123.635) (end 205.54 124.492) (width 0.25) (layer "B.Cu") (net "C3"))
 (segment (start 211.8183 126.055) (end 211.3666 125.6033) (width 0.25) (layer "B.Cu") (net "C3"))
 (segment (start 205.5375 125.7688) (end 205.4293 125.877) (width 0.25) (layer "B.Cu") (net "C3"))
 (segment (start 213.4799 123.7045) (end 210.8617 123.7045) (width 0.25) (layer "F.Cu") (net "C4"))
 (segment (start 214.3696 124.5942) (end 213.4799 123.7045) (width 0.25) (layer "F.Cu") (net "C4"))
 (via (at 214.3696 124.5942) (size 0.6) (drill 0.3) (layers "F.Cu" "B.Cu") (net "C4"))
 (via (at 210.8617 123.7045) (size 0.6) (drill 0.3) (layers "F.Cu" "B.Cu") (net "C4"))
 (segment (start 210.2198 123.7045) (end 209.2965 124.6278) (width 0.25) (layer "B.Cu") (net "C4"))
 (segment (start 207.0261 124.6278) (end 206.81 124.4117) (width 0.25) (layer "B.Cu") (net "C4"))
 (segment (start 209.2965 124.6278) (end 207.0261 124.6278) (width 0.25) (layer "B.Cu") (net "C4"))
 (segment (start 206.81 123.635) (end 206.81 124.4117) (width 0.25) (layer "B.Cu") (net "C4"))
 (segment (start 214.44 123.635) (end 214.44 124.4117) (width 0.25) (layer "B.Cu") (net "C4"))
 (segment (start 214.3697 124.5942) (end 214.3696 124.5942) (width 0.25) (layer "B.Cu") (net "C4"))
 (segment (start 210.8617 123.7045) (end 210.2198 123.7045) (width 0.25) (layer "B.Cu") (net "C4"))
 (segment (start 214.3697 124.482) (end 214.3697 124.5942) (width 0.25) (layer "B.Cu") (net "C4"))
 (segment (start 214.44 124.4117) (end 214.3697 124.482) (width 0.25) (layer "B.Cu") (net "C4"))
 (segment (start 210.1047 124.9765) (end 210.4728 124.9765) (width 0.25) (layer "F.Cu") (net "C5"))
 (segment (start 209.083 123.9548) (end 210.1047 124.9765) (width 0.25) (layer "F.Cu") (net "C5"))
 (via (at 210.4728 124.9765) (size 0.6) (drill 0.3) (layers "F.Cu" "B.Cu") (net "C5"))
 (via (at 209.083 123.9548) (size 0.6) (drill 0.3) (layers "F.Cu" "B.Cu") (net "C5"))
 (segment (start 214.6935 125.4282) (end 211.8303 125.4282) (width 0.25) (layer "B.Cu") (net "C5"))
 (segment (start 208.9067 123.7785) (end 209.083 123.9548) (width 0.25) (layer "B.Cu") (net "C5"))
 (segment (start 208.9067 123.635) (end 208.9067 123.7785) (width 0.25) (layer "B.Cu") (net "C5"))
 (segment (start 208.08 123.635) (end 208.9067 123.635) (width 0.25) (layer "B.Cu") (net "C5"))
 (segment (start 215.71 123.635) (end 215.71 124.4117) (width 0.25) (layer "B.Cu") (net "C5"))
 (segment (start 211.8303 125.4282) (end 211.3786 124.9765) (width 0.25) (layer "B.Cu") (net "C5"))
 (segment (start 211.3786 124.9765) (end 210.4728 124.9765) (width 0.25) (layer "B.Cu") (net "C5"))
 (segment (start 215.71 124.4117) (end 214.6935 125.4282) (width 0.25) (layer "B.Cu") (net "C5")))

